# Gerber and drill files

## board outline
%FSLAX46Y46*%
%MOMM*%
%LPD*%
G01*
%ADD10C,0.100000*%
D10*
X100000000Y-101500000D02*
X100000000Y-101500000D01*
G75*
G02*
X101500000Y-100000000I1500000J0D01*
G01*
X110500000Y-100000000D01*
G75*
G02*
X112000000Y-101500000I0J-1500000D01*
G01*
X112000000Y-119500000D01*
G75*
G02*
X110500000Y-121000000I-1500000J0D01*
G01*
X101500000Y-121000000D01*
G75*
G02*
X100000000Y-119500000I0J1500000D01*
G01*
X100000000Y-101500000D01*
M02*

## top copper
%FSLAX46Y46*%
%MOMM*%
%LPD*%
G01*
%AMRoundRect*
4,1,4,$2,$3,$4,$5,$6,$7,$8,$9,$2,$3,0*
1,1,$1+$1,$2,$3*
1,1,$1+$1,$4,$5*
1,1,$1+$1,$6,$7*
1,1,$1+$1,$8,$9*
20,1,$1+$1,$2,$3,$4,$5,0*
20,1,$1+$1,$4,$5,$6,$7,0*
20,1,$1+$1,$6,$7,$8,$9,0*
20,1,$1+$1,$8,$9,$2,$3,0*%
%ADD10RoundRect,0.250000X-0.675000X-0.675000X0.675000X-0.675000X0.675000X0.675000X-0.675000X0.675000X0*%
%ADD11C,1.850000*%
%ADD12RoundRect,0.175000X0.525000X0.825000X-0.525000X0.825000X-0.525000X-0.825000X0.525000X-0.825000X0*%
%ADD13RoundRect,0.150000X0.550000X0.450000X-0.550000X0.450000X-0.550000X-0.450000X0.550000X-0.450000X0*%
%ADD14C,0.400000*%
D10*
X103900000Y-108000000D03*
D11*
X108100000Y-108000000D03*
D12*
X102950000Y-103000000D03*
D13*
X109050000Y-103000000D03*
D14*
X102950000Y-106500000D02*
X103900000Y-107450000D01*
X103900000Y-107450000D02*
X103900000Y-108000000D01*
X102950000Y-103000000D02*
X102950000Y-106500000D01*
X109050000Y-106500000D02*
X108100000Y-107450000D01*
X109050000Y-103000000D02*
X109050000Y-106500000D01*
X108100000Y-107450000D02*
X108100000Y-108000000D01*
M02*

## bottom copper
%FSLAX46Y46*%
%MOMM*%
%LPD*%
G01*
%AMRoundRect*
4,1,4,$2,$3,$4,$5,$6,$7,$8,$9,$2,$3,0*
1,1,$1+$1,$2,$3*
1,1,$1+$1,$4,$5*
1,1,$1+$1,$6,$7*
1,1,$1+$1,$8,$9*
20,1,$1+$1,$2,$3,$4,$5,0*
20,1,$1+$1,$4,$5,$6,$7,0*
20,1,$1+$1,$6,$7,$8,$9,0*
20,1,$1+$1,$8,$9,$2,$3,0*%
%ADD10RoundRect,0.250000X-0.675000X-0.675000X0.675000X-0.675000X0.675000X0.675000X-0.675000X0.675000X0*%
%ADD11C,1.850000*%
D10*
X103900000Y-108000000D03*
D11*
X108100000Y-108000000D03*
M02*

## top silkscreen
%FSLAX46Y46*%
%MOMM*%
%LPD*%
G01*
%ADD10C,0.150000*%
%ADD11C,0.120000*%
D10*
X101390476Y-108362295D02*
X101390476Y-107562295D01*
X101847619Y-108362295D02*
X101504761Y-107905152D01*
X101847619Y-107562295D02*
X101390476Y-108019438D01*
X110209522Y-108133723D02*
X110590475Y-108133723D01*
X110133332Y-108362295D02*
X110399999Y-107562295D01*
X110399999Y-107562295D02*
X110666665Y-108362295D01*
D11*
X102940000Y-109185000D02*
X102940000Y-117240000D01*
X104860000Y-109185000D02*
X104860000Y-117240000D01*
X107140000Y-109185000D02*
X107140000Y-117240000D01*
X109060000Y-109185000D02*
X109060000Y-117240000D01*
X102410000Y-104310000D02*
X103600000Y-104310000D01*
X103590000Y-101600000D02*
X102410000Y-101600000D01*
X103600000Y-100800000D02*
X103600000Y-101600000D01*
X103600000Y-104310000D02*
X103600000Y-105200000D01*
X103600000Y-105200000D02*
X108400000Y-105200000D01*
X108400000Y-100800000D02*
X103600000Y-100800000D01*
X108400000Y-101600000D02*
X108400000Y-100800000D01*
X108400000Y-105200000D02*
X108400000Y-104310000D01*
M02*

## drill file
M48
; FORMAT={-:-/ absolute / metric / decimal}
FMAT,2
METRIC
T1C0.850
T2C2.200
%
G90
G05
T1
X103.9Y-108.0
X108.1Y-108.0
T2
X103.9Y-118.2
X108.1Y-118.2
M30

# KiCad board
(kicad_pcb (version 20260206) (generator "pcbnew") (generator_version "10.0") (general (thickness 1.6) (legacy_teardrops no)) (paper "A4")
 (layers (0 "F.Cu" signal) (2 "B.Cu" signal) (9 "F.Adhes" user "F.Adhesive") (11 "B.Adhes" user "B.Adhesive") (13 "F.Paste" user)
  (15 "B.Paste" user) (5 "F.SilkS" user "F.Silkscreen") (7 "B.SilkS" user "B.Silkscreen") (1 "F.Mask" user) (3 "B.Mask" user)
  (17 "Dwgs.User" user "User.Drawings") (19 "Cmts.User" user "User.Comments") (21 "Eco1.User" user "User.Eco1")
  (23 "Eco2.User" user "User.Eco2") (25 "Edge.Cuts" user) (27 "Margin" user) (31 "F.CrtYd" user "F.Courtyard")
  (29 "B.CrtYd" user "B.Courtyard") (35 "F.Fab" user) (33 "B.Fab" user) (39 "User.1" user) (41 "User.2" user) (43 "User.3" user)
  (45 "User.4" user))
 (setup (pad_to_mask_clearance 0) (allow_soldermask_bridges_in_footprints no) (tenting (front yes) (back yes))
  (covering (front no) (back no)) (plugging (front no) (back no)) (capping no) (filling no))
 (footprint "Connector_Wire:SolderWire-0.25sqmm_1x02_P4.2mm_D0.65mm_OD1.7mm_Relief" (layer "F.Cu") (at 103.9 108)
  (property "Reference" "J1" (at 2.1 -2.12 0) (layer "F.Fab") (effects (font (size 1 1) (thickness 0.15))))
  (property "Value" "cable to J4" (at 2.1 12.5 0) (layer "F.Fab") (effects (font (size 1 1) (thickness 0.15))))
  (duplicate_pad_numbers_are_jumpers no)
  (fp_line (start -0.96 1.185) (end -0.96 9.24) (stroke (width 0.12) (type solid)) (layer "F.SilkS"))
  (fp_line (start 0.96 1.185) (end 0.96 9.24) (stroke (width 0.12) (type solid)) (layer "F.SilkS"))
  (fp_line (start 3.24 1.185) (end 3.24 9.24) (stroke (width 0.12) (type solid)) (layer "F.SilkS"))
  (fp_line (start 5.16 1.185) (end 5.16 9.24) (stroke (width 0.12) (type solid)) (layer "F.SilkS"))
  (pad "" np_thru_hole circle (at 0 10.2) (size 2.2 2.2) (drill 2.2) (layers "*.Cu" "*.Mask"))
  (pad "" np_thru_hole circle (at 4.2 10.2) (size 2.2 2.2) (drill 2.2) (layers "*.Cu" "*.Mask"))
  (pad "1" thru_hole roundrect (at 0 0) (size 1.85 1.85) (drill 0.85) (layers "*.Cu" "*.Mask") (remove_unused_layers no)
   (roundrect_rratio 0.135135) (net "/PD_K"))
  (pad "2" thru_hole circle (at 4.2 0) (size 1.85 1.85) (drill 0.85) (layers "*.Cu" "*.Mask") (remove_unused_layers no) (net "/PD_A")))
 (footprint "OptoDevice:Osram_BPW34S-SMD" (layer "F.Cu") (at 106 103)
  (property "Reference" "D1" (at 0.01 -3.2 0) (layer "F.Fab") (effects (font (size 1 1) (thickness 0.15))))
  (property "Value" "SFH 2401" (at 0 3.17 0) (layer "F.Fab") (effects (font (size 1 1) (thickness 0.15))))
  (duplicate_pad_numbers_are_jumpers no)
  (fp_line (start -3.59 1.31) (end -2.4 1.31) (stroke (width 0.12) (type solid)) (layer "F.SilkS"))
  (fp_line (start -2.41 -1.4) (end -3.59 -1.4) (stroke (width 0.12) (type solid)) (layer "F.SilkS"))
  (fp_line (start -2.4 -2.2) (end -2.4 -1.4) (stroke (width 0.12) (type solid)) (layer "F.SilkS"))
  (fp_line (start -2.4 1.31) (end -2.4 2.2) (stroke (width 0.12) (type solid)) (layer "F.SilkS"))
  (fp_line (start -2.4 2.2) (end 2.4 2.2) (stroke (width 0.12) (type solid)) (layer "F.SilkS"))
  (fp_line (start 2.4 -2.2) (end -2.4 -2.2) (stroke (width 0.12) (type solid)) (layer "F.SilkS"))
  (fp_line (start 2.4 -1.4) (end 2.4 -2.2) (stroke (width 0.12) (type solid)) (layer "F.SilkS"))
  (fp_line (start 2.4 2.2) (end 2.4 1.31) (stroke (width 0.12) (type solid)) (layer "F.SilkS"))
  (pad "" smd roundrect (at -3.05 0 180) (size 1.3 1.9) (layers "F.Paste") (roundrect_rratio 0.125))
  (pad "" smd roundrect (at -3.05 0 180) (size 1.5 2.1) (layers "F.Mask") (roundrect_rratio 0.125))
  (pad "" smd roundrect (at 3.05 0 180) (size 1.3 1.1) (layers "F.Paste") (roundrect_rratio 0.125))
  (pad "" smd roundrect (at 3.05 0 180) (size 1.5 1.3) (layers "F.Mask") (roundrect_rratio 0.125))
  (pad "1" smd roundrect (at -3.05 0 180) (size 1.4 2) (layers "F.Cu" "F.Mask") (roundrect_rratio 0.125) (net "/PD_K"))
  (pad "2" smd roundrect (at 3.05 0 180) (size 1.4 1.2) (layers "F.Cu" "F.Mask") (roundrect_rratio 0.125) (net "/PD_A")))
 (gr_rect (start 100 100) (end 112 121) (radius 1.5) (stroke (width 0.1) (type solid)) (fill no) (layer "Edge.Cuts"))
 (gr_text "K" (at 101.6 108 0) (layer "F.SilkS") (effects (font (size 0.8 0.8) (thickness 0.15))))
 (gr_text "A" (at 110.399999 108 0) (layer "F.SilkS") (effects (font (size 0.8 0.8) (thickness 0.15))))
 (segment (start 102.95 106.5) (end 103.9 107.45) (width 0.4) (layer "F.Cu") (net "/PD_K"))
 (segment (start 103.9 107.45) (end 103.9 108) (width 0.4) (layer "F.Cu") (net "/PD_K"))
 (segment (start 102.95 103) (end 102.95 106.5) (width 0.4) (layer "F.Cu") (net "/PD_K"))
 (segment (start 109.05 106.5) (end 108.1 107.45) (width 0.4) (layer "F.Cu") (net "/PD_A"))
 (segment (start 109.05 103) (end 109.05 106.5) (width 0.4) (layer "F.Cu") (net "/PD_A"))
 (segment (start 108.1 107.45) (end 108.1 108) (width 0.4) (layer "F.Cu") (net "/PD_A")))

